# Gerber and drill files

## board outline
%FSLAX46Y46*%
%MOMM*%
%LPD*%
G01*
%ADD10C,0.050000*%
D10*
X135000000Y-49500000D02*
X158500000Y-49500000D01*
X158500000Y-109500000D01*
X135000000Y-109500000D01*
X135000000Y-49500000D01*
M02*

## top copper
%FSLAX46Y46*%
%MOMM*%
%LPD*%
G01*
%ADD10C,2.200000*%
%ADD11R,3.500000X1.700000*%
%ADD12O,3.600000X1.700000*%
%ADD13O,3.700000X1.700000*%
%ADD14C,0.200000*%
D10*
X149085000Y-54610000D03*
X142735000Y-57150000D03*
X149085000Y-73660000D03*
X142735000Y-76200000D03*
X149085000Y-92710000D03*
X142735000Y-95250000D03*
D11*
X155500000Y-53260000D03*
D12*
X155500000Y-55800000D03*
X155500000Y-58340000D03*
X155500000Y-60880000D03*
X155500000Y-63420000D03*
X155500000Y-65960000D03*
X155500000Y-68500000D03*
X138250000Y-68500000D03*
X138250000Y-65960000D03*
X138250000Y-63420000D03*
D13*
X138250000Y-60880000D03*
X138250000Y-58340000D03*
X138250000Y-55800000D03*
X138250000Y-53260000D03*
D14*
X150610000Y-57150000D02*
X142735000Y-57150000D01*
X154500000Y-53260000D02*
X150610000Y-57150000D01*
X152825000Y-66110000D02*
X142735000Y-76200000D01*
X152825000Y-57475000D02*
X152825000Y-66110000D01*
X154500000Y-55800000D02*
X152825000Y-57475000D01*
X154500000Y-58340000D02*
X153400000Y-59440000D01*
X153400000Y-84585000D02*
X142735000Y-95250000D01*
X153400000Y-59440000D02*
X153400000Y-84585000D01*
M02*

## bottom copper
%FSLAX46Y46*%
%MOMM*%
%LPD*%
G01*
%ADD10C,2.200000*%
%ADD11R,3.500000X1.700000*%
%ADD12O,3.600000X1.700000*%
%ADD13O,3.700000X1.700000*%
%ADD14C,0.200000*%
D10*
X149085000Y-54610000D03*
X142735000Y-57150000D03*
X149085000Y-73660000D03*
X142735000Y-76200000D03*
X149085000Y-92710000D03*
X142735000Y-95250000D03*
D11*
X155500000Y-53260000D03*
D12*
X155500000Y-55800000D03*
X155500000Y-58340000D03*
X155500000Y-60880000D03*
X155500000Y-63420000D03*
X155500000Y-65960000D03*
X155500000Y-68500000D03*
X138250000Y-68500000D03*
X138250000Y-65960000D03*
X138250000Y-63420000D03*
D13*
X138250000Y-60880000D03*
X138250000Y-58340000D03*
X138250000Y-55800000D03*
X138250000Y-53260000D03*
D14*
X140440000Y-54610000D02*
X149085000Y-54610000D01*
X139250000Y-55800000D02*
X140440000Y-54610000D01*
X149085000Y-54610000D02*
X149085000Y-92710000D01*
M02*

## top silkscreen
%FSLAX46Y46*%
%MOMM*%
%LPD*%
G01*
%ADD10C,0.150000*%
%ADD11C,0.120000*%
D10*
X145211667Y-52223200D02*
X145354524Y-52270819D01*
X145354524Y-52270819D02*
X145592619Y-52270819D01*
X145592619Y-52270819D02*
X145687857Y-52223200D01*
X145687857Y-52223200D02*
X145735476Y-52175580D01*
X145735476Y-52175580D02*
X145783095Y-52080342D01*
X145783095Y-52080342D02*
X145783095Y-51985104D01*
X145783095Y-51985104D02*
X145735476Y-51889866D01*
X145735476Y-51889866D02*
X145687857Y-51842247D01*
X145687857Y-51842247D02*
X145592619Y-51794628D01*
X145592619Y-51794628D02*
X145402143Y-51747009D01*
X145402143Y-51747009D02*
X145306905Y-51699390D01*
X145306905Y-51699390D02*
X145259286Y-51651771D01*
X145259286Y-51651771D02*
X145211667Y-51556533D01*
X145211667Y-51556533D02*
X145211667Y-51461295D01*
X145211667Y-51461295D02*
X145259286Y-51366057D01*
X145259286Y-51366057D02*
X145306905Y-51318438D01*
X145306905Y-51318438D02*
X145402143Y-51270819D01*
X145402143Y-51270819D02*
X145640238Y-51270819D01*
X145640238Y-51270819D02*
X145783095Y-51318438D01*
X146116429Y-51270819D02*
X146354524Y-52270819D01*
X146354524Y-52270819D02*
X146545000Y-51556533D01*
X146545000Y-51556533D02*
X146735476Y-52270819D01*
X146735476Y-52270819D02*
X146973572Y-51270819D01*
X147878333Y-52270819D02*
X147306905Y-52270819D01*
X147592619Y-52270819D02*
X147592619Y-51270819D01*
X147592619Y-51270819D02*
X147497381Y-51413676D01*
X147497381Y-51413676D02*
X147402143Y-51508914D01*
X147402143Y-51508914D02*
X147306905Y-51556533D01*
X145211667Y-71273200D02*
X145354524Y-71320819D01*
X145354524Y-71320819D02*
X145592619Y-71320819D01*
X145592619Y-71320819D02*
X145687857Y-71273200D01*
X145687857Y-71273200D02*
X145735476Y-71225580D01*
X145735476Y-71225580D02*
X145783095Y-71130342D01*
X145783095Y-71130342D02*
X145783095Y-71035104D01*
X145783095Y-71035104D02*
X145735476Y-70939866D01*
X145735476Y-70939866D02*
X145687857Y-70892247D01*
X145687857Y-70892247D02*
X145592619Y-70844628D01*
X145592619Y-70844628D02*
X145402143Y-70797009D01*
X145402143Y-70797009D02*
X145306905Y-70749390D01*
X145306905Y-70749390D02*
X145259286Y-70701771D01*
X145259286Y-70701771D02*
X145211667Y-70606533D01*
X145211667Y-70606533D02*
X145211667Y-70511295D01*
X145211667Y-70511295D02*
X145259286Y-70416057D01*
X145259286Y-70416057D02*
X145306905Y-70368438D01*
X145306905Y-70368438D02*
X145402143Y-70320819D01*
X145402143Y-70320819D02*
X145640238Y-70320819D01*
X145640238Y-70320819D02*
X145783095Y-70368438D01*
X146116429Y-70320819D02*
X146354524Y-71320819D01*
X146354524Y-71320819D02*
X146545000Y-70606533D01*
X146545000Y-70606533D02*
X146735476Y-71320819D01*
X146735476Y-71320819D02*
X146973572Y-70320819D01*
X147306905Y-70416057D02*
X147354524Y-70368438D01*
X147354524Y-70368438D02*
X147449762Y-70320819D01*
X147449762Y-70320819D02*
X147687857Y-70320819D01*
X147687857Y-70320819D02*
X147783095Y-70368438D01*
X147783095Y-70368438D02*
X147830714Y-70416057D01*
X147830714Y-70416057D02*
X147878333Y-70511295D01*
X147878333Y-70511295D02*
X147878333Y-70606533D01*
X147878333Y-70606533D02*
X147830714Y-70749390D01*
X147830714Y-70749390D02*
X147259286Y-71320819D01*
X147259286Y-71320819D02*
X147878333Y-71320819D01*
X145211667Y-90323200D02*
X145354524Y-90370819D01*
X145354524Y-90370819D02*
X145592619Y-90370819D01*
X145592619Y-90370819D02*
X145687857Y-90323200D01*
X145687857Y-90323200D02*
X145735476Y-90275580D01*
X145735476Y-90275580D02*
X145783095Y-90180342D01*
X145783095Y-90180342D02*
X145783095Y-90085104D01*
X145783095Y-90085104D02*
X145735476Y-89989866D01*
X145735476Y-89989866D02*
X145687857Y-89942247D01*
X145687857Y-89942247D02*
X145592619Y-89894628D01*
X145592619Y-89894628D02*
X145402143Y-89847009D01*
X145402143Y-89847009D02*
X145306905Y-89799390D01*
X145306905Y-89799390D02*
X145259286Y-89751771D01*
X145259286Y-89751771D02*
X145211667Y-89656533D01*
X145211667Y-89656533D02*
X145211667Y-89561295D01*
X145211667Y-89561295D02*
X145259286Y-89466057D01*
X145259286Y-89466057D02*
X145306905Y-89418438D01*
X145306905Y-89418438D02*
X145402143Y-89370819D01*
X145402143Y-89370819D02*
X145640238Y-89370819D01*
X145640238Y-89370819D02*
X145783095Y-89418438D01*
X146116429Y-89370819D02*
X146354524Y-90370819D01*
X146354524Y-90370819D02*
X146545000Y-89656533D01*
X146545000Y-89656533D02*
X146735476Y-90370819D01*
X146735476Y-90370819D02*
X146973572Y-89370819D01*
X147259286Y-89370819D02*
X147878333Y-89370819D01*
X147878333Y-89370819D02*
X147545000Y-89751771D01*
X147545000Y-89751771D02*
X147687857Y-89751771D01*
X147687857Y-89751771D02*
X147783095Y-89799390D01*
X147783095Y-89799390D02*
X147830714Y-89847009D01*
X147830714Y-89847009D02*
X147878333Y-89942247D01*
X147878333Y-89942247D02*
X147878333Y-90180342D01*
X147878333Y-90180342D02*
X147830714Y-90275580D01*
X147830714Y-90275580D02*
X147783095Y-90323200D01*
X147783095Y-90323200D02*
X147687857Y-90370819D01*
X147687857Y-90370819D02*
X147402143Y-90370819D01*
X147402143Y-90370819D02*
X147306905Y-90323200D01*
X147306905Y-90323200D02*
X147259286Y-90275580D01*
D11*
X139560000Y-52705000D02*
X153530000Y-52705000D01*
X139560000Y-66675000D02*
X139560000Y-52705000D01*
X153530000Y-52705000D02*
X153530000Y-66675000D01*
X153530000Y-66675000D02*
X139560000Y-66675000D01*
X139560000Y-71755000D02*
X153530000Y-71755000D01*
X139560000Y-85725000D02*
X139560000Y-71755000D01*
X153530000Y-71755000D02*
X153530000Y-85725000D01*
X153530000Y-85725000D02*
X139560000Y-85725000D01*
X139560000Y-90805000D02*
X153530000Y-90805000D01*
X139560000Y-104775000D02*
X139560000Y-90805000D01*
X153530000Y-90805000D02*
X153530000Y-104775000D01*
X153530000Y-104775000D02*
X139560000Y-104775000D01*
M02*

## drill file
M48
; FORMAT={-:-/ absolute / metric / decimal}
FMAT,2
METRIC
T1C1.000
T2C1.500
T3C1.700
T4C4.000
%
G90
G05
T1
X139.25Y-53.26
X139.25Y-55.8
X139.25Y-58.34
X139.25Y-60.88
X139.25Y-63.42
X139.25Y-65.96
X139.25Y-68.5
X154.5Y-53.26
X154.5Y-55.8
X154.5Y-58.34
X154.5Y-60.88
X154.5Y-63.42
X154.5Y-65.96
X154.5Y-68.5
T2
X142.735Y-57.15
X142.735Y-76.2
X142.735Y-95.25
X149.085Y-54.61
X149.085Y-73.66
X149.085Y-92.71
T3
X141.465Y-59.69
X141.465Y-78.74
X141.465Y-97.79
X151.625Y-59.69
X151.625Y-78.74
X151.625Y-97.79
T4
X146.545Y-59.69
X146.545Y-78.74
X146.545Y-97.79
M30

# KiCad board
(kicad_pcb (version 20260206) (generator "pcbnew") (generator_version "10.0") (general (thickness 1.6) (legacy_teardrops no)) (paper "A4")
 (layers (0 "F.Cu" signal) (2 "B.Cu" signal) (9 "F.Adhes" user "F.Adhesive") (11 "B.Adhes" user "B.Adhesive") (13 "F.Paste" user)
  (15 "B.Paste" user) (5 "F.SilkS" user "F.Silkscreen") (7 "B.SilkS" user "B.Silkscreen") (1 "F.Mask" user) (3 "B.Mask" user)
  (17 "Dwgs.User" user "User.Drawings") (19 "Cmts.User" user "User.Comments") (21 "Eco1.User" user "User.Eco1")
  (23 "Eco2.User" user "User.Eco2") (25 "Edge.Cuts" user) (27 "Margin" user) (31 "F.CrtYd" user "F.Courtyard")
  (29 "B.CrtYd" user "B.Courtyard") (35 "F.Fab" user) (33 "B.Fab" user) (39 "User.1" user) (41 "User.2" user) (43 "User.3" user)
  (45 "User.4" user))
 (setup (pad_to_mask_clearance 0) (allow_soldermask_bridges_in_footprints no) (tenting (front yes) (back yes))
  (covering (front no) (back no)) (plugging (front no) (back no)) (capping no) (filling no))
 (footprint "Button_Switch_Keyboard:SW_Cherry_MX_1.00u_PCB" (layer "F.Cu") (at 149.085 54.61)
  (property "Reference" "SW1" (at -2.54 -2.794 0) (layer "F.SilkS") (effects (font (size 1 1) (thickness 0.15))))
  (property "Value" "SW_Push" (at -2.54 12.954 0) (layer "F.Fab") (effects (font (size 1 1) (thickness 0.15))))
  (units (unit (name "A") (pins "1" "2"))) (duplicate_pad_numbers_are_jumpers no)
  (fp_line (start -9.525 -1.905) (end 4.445 -1.905) (stroke (width 0.12) (type solid)) (layer "F.SilkS"))
  (fp_line (start -9.525 12.065) (end -9.525 -1.905) (stroke (width 0.12) (type solid)) (layer "F.SilkS"))
  (fp_line (start 4.445 -1.905) (end 4.445 12.065) (stroke (width 0.12) (type solid)) (layer "F.SilkS"))
  (fp_line (start 4.445 12.065) (end -9.525 12.065) (stroke (width 0.12) (type solid)) (layer "F.SilkS"))
  (pad "" np_thru_hole circle (at -7.62 5.08) (size 1.7 1.7) (drill 1.7) (layers "*.Cu" "*.Mask"))
  (pad "" np_thru_hole circle (at -2.54 5.08) (size 4 4) (drill 4) (layers "*.Cu" "*.Mask"))
  (pad "" np_thru_hole circle (at 2.54 5.08) (size 1.7 1.7) (drill 1.7) (layers "*.Cu" "*.Mask"))
  (pad "1" thru_hole circle (at 0 0) (size 2.2 2.2) (drill 1.5) (layers "*.Cu" "*.Mask") (remove_unused_layers no) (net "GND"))
  (pad "2" thru_hole circle (at -6.35 2.54) (size 2.2 2.2) (drill 1.5) (layers "*.Cu" "*.Mask") (remove_unused_layers no)
   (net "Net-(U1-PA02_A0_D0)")))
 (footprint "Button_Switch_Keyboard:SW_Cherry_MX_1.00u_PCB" (layer "F.Cu") (at 149.085 73.66)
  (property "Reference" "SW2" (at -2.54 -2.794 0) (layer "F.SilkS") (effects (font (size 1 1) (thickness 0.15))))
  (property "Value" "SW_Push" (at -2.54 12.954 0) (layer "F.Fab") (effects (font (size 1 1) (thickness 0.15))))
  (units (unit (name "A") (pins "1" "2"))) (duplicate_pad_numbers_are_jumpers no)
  (fp_line (start -9.525 -1.905) (end 4.445 -1.905) (stroke (width 0.12) (type solid)) (layer "F.SilkS"))
  (fp_line (start -9.525 12.065) (end -9.525 -1.905) (stroke (width 0.12) (type solid)) (layer "F.SilkS"))
  (fp_line (start 4.445 -1.905) (end 4.445 12.065) (stroke (width 0.12) (type solid)) (layer "F.SilkS"))
  (fp_line (start 4.445 12.065) (end -9.525 12.065) (stroke (width 0.12) (type solid)) (layer "F.SilkS"))
  (pad "" np_thru_hole circle (at -7.62 5.08) (size 1.7 1.7) (drill 1.7) (layers "*.Cu" "*.Mask"))
  (pad "" np_thru_hole circle (at -2.54 5.08) (size 4 4) (drill 4) (layers "*.Cu" "*.Mask"))
  (pad "" np_thru_hole circle (at 2.54 5.08) (size 1.7 1.7) (drill 1.7) (layers "*.Cu" "*.Mask"))
  (pad "1" thru_hole circle (at 0 0) (size 2.2 2.2) (drill 1.5) (layers "*.Cu" "*.Mask") (remove_unused_layers no) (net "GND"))
  (pad "2" thru_hole circle (at -6.35 2.54) (size 2.2 2.2) (drill 1.5) (layers "*.Cu" "*.Mask") (remove_unused_layers no)
   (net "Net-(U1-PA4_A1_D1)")))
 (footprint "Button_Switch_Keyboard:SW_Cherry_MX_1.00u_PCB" (layer "F.Cu") (at 149.085 92.71)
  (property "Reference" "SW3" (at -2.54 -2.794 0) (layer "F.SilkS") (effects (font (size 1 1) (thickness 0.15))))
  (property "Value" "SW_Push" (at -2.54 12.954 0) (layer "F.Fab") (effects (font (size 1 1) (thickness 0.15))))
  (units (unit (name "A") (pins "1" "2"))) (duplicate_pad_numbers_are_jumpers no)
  (fp_line (start -9.525 -1.905) (end 4.445 -1.905) (stroke (width 0.12) (type solid)) (layer "F.SilkS"))
  (fp_line (start -9.525 12.065) (end -9.525 -1.905) (stroke (width 0.12) (type solid)) (layer "F.SilkS"))
  (fp_line (start 4.445 -1.905) (end 4.445 12.065) (stroke (width 0.12) (type solid)) (layer "F.SilkS"))
  (fp_line (start 4.445 12.065) (end -9.525 12.065) (stroke (width 0.12) (type solid)) (layer "F.SilkS"))
  (pad "" np_thru_hole circle (at -7.62 5.08) (size 1.7 1.7) (drill 1.7) (layers "*.Cu" "*.Mask"))
  (pad "" np_thru_hole circle (at -2.54 5.08) (size 4 4) (drill 4) (layers "*.Cu" "*.Mask"))
  (pad "" np_thru_hole circle (at 2.54 5.08) (size 1.7 1.7) (drill 1.7) (layers "*.Cu" "*.Mask"))
  (pad "1" thru_hole circle (at 0 0) (size 2.2 2.2) (drill 1.5) (layers "*.Cu" "*.Mask") (remove_unused_layers no) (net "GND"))
  (pad "2" thru_hole circle (at -6.35 2.54) (size 2.2 2.2) (drill 1.5) (layers "*.Cu" "*.Mask") (remove_unused_layers no)
   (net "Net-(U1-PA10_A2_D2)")))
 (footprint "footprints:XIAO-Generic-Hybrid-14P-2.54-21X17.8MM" (layer "B.Cu") (at 146.875 60.88 180)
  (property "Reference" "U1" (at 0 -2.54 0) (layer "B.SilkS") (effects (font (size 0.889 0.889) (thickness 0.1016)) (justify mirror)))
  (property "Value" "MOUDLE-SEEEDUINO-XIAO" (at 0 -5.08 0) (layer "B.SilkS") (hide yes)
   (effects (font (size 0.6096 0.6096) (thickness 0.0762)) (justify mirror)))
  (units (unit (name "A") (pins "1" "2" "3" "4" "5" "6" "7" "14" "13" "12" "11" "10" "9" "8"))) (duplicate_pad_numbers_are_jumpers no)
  (pad "1" thru_hole rect (at -7.625 7.62 180) (size 3.5 1.7) (drill 1 (offset -1 0)) (layers "*.Cu" "*.Mask") (remove_unused_layers no)
   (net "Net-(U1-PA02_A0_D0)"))
  (pad "2" thru_hole oval (at -7.625 5.08 180) (size 3.6 1.7) (drill 1 (offset -1 0)) (layers "*.Cu" "*.Mask") (remove_unused_layers no)
   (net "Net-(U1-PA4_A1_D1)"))
  (pad "3" thru_hole oval (at -7.625 2.54 180) (size 3.6 1.7) (drill 1 (offset -1 0)) (layers "*.Cu" "*.Mask") (remove_unused_layers no)
   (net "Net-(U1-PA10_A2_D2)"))
  (pad "4" thru_hole oval (at -7.625 0 180) (size 3.6 1.7) (drill 1 (offset -1 0)) (layers "*.Cu" "*.Mask") (remove_unused_layers no)
   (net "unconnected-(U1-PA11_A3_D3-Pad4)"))
  (pad "5" thru_hole oval (at -7.625 -2.54 180) (size 3.6 1.7) (drill 1 (offset -1 0)) (layers "*.Cu" "*.Mask") (remove_unused_layers no)
   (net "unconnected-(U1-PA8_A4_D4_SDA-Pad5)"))
  (pad "6" thru_hole oval (at -7.625 -5.08) (size 3.6 1.7) (drill 1 (offset 1 0)) (layers "*.Cu" "*.Mask") (remove_unused_layers no)
   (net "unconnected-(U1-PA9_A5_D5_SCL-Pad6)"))
  (pad "7" thru_hole oval (at -7.625 -7.62 180) (size 3.6 1.7) (drill 1 (offset -1 0)) (layers "*.Cu" "*.Mask") (remove_unused_layers no)
   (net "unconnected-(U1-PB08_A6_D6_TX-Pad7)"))
  (pad "8" thru_hole oval (at 7.625 -7.62 180) (size 3.6 1.7) (drill 1 (offset 1 0)) (layers "*.Cu" "*.Mask") (remove_unused_layers no)
   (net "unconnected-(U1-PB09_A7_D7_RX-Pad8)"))
  (pad "9" thru_hole oval (at 7.625 -5.08 180) (size 3.6 1.7) (drill 1 (offset 1 0)) (layers "*.Cu" "*.Mask") (remove_unused_layers no)
   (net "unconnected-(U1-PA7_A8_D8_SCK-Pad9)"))
  (pad "10" thru_hole oval (at 7.625 -2.54 180) (size 3.6 1.7) (drill 1 (offset 1 0)) (layers "*.Cu" "*.Mask") (remove_unused_layers no)
   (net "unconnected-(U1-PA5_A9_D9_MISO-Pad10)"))
  (pad "11" thru_hole oval (at 7.625 0 180) (size 3.7 1.7) (drill 1 (offset 1 0)) (layers "*.Cu" "*.Mask") (remove_unused_layers no)
   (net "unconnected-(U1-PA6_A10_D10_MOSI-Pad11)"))
  (pad "12" thru_hole oval (at 7.625 2.54 180) (size 3.7 1.7) (drill 1 (offset 1 0)) (layers "*.Cu" "*.Mask") (remove_unused_layers no)
   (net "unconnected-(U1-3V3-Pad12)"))
  (pad "13" thru_hole oval (at 7.625 5.08 180) (size 3.7 1.7) (drill 1 (offset 1 0)) (layers "*.Cu" "*.Mask") (remove_unused_layers no)
   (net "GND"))
  (pad "14" thru_hole oval (at 7.625 7.62 180) (size 3.7 1.7) (drill 1 (offset 1 0)) (layers "*.Cu" "*.Mask") (remove_unused_layers no)
   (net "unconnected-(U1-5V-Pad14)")))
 (gr_rect (start 135 49.5) (end 158.5 109.5) (stroke (width 0.05) (type default)) (fill no) (layer "Edge.Cuts"))
 (segment (start 140.44 54.61) (end 149.085 54.61) (width 0.2) (layer "B.Cu") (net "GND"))
 (segment (start 139.25 55.8) (end 140.44 54.61) (width 0.2) (layer "B.Cu") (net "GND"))
 (segment (start 149.085 54.61) (end 149.085 92.71) (width 0.2) (layer "B.Cu") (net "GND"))
 (segment (start 150.61 57.15) (end 142.735 57.15) (width 0.2) (layer "F.Cu") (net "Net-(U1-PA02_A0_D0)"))
 (segment (start 154.5 53.26) (end 150.61 57.15) (width 0.2) (layer "F.Cu") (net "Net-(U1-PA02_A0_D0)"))
 (segment (start 152.825 66.11) (end 142.735 76.2) (width 0.2) (layer "F.Cu") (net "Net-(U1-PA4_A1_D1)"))
 (segment (start 152.825 57.475) (end 152.825 66.11) (width 0.2) (layer "F.Cu") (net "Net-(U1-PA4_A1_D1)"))
 (segment (start 154.5 55.8) (end 152.825 57.475) (width 0.2) (layer "F.Cu") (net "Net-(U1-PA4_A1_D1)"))
 (segment (start 154.5 58.34) (end 153.4 59.44) (width 0.2) (layer "F.Cu") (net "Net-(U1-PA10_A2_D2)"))
 (segment (start 153.4 84.585) (end 142.735 95.25) (width 0.2) (layer "F.Cu") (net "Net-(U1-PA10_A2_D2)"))
 (segment (start 153.4 59.44) (end 153.4 84.585) (width 0.2) (layer "F.Cu") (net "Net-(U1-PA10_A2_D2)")))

